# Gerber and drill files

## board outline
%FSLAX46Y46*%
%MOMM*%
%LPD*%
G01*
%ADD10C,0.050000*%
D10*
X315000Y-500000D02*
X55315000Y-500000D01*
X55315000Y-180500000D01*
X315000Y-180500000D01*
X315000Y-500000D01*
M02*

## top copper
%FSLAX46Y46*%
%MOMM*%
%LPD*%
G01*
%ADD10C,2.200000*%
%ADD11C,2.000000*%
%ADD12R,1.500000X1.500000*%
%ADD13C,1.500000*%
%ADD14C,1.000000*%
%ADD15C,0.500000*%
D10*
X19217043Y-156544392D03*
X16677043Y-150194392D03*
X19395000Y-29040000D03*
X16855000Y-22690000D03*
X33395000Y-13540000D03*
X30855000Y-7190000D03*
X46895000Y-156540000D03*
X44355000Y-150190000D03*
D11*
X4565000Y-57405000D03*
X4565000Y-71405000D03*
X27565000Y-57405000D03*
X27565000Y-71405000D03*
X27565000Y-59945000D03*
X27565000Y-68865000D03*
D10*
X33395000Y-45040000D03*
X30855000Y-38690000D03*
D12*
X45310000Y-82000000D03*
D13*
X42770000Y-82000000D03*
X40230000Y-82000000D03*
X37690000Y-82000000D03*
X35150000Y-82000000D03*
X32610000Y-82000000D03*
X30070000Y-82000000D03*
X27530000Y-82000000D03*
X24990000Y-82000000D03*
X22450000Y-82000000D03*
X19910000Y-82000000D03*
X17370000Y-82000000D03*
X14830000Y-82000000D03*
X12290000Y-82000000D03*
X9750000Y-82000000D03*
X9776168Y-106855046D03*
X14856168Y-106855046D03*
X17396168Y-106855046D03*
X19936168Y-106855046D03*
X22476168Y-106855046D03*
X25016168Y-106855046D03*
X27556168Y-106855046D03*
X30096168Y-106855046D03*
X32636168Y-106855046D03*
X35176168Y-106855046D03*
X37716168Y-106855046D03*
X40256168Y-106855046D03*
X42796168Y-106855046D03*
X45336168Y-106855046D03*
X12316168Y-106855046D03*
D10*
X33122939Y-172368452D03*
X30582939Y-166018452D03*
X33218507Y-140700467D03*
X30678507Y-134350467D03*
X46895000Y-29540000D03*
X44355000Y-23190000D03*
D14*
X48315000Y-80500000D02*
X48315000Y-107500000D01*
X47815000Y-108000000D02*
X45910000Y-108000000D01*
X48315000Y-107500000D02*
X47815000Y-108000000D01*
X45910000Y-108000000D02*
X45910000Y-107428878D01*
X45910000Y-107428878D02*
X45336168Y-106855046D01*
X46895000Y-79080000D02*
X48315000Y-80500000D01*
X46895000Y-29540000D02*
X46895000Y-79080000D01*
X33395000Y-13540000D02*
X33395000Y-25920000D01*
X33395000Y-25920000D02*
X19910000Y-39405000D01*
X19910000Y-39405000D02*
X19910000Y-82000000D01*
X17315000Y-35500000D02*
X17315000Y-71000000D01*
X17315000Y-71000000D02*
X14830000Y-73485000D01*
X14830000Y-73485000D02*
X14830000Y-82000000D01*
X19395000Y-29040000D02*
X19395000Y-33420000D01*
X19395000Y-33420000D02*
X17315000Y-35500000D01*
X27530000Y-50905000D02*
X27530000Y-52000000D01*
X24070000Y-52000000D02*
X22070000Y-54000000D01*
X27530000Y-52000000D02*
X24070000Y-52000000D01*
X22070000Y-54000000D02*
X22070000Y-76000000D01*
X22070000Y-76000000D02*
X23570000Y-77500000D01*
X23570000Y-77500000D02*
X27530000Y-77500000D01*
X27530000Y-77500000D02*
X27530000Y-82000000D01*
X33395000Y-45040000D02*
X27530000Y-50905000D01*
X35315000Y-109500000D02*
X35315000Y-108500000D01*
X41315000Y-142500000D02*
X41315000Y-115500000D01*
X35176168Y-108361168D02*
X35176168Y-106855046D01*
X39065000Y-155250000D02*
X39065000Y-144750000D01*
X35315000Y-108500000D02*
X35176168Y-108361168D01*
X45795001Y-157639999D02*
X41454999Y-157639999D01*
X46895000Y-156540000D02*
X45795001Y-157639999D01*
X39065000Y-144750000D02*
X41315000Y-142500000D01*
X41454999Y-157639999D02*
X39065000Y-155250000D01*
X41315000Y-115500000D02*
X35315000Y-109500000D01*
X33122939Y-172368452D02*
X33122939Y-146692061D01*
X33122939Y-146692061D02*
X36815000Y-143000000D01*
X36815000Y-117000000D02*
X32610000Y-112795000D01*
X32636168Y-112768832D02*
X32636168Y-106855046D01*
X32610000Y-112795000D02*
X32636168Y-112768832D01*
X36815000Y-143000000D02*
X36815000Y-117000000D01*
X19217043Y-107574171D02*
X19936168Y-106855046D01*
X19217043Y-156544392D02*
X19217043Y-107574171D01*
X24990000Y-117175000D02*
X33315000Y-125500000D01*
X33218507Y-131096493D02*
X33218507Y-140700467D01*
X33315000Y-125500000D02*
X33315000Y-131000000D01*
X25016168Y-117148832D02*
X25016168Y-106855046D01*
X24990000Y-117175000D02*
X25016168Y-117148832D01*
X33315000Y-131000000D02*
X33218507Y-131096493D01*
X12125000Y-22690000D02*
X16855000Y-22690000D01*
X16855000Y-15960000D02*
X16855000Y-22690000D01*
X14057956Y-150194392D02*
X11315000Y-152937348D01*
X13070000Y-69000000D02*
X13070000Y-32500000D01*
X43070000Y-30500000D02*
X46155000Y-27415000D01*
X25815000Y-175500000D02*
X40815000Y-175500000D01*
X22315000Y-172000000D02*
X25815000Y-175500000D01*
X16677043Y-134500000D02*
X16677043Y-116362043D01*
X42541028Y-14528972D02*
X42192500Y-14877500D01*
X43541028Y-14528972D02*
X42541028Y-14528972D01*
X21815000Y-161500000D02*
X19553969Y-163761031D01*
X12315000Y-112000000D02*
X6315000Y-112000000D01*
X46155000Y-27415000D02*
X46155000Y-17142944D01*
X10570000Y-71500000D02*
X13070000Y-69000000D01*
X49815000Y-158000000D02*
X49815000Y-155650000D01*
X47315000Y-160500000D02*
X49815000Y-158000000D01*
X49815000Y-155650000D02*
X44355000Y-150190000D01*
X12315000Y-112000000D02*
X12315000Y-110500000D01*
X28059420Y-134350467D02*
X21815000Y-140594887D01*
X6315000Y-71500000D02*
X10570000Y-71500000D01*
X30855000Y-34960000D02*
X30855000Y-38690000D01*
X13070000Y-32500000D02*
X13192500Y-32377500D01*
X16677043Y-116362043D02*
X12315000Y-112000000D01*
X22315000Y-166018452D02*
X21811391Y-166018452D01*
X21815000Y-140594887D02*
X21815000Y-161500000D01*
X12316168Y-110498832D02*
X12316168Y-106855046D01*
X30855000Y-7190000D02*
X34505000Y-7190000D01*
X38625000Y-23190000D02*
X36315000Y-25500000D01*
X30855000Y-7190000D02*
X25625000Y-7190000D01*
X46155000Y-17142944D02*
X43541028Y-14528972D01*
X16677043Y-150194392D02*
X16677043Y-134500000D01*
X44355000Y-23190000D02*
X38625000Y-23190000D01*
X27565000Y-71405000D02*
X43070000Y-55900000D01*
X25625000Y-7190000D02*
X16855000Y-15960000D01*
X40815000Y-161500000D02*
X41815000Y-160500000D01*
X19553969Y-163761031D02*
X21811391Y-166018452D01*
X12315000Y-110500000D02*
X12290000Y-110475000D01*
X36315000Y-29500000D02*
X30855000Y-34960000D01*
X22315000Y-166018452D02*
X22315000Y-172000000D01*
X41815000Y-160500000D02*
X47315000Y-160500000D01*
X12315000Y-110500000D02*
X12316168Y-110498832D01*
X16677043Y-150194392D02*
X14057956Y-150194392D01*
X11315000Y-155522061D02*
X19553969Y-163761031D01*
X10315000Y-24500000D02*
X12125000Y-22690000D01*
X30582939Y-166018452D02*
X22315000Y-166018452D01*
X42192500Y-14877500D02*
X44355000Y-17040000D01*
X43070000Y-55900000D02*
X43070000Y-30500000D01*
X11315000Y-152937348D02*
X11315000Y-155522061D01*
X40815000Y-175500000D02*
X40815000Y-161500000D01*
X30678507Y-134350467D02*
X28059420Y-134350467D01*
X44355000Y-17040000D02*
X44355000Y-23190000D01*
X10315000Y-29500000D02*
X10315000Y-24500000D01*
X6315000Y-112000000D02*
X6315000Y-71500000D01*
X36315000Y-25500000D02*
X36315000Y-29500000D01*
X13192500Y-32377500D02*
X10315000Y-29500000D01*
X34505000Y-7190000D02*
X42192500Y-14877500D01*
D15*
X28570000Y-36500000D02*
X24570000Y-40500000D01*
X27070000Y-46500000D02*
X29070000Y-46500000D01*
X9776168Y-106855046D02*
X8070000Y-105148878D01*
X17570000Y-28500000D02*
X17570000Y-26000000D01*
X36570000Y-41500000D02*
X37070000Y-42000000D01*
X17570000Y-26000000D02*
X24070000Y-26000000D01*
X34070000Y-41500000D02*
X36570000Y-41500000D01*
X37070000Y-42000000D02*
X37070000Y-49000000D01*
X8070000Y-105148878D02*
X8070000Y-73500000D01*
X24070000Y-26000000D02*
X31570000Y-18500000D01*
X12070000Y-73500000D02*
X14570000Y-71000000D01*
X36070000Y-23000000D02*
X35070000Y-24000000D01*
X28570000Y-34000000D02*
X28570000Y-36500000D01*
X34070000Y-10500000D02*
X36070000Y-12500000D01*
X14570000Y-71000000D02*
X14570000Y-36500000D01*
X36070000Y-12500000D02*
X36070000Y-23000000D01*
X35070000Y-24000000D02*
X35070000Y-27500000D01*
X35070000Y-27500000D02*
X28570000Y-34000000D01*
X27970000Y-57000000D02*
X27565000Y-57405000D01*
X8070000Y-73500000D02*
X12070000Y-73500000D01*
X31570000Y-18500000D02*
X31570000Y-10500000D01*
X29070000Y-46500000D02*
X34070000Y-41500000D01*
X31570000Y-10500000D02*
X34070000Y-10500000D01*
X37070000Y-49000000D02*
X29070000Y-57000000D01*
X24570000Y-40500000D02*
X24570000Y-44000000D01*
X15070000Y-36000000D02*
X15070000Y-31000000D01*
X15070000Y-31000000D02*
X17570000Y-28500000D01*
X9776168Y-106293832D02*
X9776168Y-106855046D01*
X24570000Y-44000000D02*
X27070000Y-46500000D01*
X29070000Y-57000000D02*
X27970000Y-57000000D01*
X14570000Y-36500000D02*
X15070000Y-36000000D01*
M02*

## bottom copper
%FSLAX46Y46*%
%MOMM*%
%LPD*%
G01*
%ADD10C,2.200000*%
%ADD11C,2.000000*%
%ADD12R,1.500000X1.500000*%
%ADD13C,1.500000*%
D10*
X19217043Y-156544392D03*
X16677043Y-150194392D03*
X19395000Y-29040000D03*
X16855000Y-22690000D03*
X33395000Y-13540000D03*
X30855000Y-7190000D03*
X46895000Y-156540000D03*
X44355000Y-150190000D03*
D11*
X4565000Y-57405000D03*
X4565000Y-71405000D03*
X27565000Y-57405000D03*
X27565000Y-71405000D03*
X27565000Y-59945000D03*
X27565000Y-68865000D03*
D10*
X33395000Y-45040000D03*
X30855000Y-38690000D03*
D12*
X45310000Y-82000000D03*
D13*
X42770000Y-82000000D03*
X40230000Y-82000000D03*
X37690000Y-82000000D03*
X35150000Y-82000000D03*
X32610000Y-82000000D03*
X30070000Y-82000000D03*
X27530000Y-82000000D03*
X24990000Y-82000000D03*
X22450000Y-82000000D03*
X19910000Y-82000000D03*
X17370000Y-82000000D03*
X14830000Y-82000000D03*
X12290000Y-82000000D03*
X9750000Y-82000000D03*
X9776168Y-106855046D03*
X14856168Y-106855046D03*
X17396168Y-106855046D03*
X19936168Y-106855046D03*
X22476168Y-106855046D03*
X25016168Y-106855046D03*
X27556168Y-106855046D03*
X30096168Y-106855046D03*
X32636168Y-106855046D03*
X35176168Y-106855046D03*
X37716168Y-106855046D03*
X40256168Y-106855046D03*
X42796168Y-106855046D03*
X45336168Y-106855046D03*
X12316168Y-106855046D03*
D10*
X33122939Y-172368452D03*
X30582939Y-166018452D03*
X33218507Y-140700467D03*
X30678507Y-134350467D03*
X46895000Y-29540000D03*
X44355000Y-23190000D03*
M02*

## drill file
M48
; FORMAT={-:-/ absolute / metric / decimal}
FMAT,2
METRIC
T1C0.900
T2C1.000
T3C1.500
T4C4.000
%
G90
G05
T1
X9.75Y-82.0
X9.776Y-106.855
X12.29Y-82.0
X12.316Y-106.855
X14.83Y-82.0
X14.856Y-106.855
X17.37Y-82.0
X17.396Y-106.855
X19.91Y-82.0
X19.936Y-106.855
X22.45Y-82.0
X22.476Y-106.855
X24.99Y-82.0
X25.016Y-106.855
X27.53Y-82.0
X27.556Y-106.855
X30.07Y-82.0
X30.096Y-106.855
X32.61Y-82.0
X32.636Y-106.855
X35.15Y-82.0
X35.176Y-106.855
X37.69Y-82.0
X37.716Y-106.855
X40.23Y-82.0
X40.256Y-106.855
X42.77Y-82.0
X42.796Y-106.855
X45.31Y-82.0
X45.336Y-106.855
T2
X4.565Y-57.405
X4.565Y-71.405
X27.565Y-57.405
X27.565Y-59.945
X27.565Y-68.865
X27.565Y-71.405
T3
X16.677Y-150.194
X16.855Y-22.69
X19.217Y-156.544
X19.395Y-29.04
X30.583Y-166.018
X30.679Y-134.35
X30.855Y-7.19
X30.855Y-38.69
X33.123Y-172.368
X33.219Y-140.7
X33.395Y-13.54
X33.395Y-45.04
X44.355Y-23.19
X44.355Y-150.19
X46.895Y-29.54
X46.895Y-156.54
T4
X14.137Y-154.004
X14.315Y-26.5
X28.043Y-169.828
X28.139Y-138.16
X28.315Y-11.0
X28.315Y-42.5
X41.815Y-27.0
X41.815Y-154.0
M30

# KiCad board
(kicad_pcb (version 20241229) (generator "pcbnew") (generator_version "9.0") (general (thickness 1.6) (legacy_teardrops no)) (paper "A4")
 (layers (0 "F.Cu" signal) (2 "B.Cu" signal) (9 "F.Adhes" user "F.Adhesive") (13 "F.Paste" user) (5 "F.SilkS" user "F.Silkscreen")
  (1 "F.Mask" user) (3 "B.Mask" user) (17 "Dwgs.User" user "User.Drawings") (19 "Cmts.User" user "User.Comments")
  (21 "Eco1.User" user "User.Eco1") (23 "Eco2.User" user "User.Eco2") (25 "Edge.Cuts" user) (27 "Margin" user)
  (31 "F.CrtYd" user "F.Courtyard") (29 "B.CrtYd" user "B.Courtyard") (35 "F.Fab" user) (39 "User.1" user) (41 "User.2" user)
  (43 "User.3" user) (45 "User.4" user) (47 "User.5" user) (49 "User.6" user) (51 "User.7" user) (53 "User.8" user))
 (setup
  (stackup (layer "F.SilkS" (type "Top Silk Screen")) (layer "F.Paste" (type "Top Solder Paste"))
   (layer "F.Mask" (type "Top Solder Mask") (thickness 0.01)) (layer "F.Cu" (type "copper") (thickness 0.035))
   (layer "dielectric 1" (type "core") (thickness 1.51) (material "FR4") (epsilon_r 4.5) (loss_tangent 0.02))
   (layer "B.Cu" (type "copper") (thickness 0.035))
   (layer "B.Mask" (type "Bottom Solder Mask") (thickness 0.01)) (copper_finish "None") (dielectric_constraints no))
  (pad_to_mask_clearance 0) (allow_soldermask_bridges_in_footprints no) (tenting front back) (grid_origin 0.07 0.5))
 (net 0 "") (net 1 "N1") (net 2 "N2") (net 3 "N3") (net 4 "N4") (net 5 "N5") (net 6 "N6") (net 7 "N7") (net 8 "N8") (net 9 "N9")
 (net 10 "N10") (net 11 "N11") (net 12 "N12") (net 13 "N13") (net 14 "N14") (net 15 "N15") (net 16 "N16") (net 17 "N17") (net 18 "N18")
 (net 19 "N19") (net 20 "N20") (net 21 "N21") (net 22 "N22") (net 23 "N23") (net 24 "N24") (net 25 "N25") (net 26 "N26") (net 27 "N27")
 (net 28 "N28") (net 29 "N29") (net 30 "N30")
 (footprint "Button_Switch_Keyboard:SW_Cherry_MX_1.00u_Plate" (layer "F.Cu") (at 19.217043 156.544392 -90)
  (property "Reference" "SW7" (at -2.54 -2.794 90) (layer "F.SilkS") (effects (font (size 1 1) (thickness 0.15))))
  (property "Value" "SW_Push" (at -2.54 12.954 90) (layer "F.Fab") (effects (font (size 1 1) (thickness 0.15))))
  (pad "" np_thru_hole circle (at -2.54 5.08 270) (size 4 4) (drill 4) (layers "*.Cu" "*.Mask"))
  (pad "1" thru_hole circle (at 0 0 270) (size 2.2 2.2) (drill 1.5) (layers "*.Cu" "*.Mask") (remove_unused_layers no) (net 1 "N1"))
  (pad "2" thru_hole circle (at -6.35 2.54 270) (size 2.2 2.2) (drill 1.5) (layers "*.Cu" "*.Mask") (remove_unused_layers no) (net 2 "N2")))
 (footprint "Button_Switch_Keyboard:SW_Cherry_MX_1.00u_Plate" (layer "F.Cu") (at 19.395 29.04 -90)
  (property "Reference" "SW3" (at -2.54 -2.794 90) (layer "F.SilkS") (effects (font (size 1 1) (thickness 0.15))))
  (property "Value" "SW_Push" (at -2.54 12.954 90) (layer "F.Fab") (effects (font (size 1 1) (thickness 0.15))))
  (pad "" np_thru_hole circle (at -2.54 5.08 270) (size 4 4) (drill 4) (layers "*.Cu" "*.Mask"))
  (pad "1" thru_hole circle (at 0 0 270) (size 2.2 2.2) (drill 1.5) (layers "*.Cu" "*.Mask") (remove_unused_layers no) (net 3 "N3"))
  (pad "2" thru_hole circle (at -6.35 2.54 270) (size 2.2 2.2) (drill 1.5) (layers "*.Cu" "*.Mask") (remove_unused_layers no) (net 2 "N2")))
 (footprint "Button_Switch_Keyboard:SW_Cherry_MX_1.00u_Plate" (layer "F.Cu") (at 33.395 13.54 -90)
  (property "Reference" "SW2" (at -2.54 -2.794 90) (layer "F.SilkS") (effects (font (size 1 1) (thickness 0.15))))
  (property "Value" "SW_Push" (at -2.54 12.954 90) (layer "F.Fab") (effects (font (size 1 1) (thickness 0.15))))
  (pad "" np_thru_hole circle (at -2.54 5.08 270) (size 4 4) (drill 4) (layers "*.Cu" "*.Mask"))
  (pad "1" thru_hole circle (at 0 0 270) (size 2.2 2.2) (drill 1.5) (layers "*.Cu" "*.Mask") (remove_unused_layers no) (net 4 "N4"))
  (pad "2" thru_hole circle (at -6.35 2.54 270) (size 2.2 2.2) (drill 1.5) (layers "*.Cu" "*.Mask") (remove_unused_layers no) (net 2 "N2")))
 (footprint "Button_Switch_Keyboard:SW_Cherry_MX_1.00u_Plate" (layer "F.Cu") (at 46.895 156.54 -90)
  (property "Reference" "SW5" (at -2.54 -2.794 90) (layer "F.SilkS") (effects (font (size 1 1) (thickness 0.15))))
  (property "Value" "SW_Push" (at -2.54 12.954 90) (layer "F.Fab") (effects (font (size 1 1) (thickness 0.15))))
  (pad "" np_thru_hole circle (at -2.54 5.08 270) (size 4 4) (drill 4) (layers "*.Cu" "*.Mask"))
  (pad "1" thru_hole circle (at 0 0 270) (size 2.2 2.2) (drill 1.5) (layers "*.Cu" "*.Mask") (remove_unused_layers no) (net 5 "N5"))
  (pad "2" thru_hole circle (at -6.35 2.54 270) (size 2.2 2.2) (drill 1.5) (layers "*.Cu" "*.Mask") (remove_unused_layers no) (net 2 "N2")))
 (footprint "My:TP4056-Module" (layer "F.Cu") (at 2.065 73.005)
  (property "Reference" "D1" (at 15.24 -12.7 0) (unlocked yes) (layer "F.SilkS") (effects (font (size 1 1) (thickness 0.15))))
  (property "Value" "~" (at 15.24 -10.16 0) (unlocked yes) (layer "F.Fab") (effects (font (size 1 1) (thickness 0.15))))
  (pad "1" thru_hole circle (at 2.5 -15.6) (size 2 2) (drill 1) (layers "*.Cu" "*.Mask") (remove_unused_layers no))
  (pad "2" thru_hole circle (at 2.5 -1.6) (size 2 2) (drill 1) (layers "*.Cu" "*.Mask") (remove_unused_layers no))
  (pad "3" thru_hole circle (at 25.5 -15.6) (size 2 2) (drill 1) (layers "*.Cu" "*.Mask") (remove_unused_layers no) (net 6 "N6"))
  (pad "4" thru_hole circle (at 25.5 -1.6) (size 2 2) (drill 1) (layers "*.Cu" "*.Mask") (remove_unused_layers no) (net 2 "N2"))
  (pad "5" thru_hole circle (at 25.5 -13.06) (size 2 2) (drill 1) (layers "*.Cu" "*.Mask") (remove_unused_layers no))
  (pad "6" thru_hole circle (at 25.5 -4.14) (size 2 2) (drill 1) (layers "*.Cu" "*.Mask") (remove_unused_layers no)))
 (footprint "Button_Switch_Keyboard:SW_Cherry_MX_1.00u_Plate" (layer "F.Cu") (at 33.395 45.04 -90)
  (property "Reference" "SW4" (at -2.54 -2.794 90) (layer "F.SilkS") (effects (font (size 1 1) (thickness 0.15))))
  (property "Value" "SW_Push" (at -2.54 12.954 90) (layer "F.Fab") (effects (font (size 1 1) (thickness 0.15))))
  (pad "" np_thru_hole circle (at -2.54 5.08 270) (size 4 4) (drill 4) (layers "*.Cu" "*.Mask"))
  (pad "1" thru_hole circle (at 0 0 270) (size 2.2 2.2) (drill 1.5) (layers "*.Cu" "*.Mask") (remove_unused_layers no) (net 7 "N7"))
  (pad "2" thru_hole circle (at -6.35 2.54 270) (size 2.2 2.2) (drill 1.5) (layers "*.Cu" "*.Mask") (remove_unused_layers no) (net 2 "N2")))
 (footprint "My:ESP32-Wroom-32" (layer "F.Cu") (at 45.31 82 -90)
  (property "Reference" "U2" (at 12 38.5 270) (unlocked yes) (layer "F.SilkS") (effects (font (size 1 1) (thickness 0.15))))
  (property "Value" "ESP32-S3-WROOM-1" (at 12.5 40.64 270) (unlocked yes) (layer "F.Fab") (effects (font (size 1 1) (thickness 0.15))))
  (pad "1" thru_hole rect (at 0 0 270) (size 1.5 1.5) (drill 0.9) (layers "*.Cu" "*.Mask") (remove_unused_layers yes) (keep_end_layers yes)
   (zone_layer_connections) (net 2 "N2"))
  (pad "2" thru_hole circle (at 0 2.54 270) (size 1.5 1.5) (drill 0.9) (layers "*.Cu" "*.Mask") (remove_unused_layers yes)
   (keep_end_layers yes) (zone_layer_connections) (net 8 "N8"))
  (pad "3" thru_hole circle (at 0 5.08 270) (size 1.5 1.5) (drill 0.9) (layers "*.Cu" "*.Mask") (remove_unused_layers yes)
   (keep_end_layers yes) (zone_layer_connections) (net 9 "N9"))
  (pad "4" thru_hole circle (at 0 7.62 270) (size 1.5 1.5) (drill 0.9) (layers "*.Cu" "*.Mask") (remove_unused_layers yes)
   (keep_end_layers yes) (zone_layer_connections) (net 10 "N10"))
  (pad "5" thru_hole circle (at 0 10.16 270) (size 1.5 1.5) (drill 0.9) (layers "*.Cu" "*.Mask") (remove_unused_layers yes)
   (keep_end_layers yes) (zone_layer_connections) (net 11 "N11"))
  (pad "6" thru_hole circle (at 0 12.7 270) (size 1.5 1.5) (drill 0.9) (layers "*.Cu" "*.Mask") (remove_unused_layers yes)
   (keep_end_layers yes) (zone_layer_connections) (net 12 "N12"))
  (pad "7" thru_hole circle (at 0 15.24 270) (size 1.5 1.5) (drill 0.9) (layers "*.Cu" "*.Mask") (remove_unused_layers yes)
   (keep_end_layers yes) (zone_layer_connections) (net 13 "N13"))
  (pad "8" thru_hole circle (at 0 17.78 270) (size 1.5 1.5) (drill 0.9) (layers "*.Cu" "*.Mask") (remove_unused_layers yes)
   (keep_end_layers yes) (zone_layer_connections) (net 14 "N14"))
  (pad "9" thru_hole circle (at 0 20.32 270) (size 1.5 1.5) (drill 0.9) (layers "*.Cu" "*.Mask") (remove_unused_layers yes)
   (keep_end_layers yes) (zone_layer_connections) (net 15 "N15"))
  (pad "10" thru_hole circle (at 0 22.86 270) (size 1.5 1.5) (drill 0.9) (layers "*.Cu" "*.Mask") (remove_unused_layers yes)
   (keep_end_layers yes) (zone_layer_connections) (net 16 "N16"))
  (pad "11" thru_hole circle (at 0 25.4 270) (size 1.5 1.5) (drill 0.9) (layers "*.Cu" "*.Mask") (remove_unused_layers yes)
   (keep_end_layers yes) (zone_layer_connections) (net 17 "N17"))
  (pad "12" thru_hole circle (at 0 27.94 270) (size 1.5 1.5) (drill 0.9) (layers "*.Cu" "*.Mask") (remove_unused_layers yes)
   (keep_end_layers yes) (zone_layer_connections) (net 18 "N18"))
  (pad "13" thru_hole circle (at 0 30.48 270) (size 1.5 1.5) (drill 0.9) (layers "*.Cu" "*.Mask") (remove_unused_layers yes)
   (keep_end_layers yes) (zone_layer_connections) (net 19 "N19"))
  (pad "14" thru_hole circle (at 0 33.02 270) (size 1.5 1.5) (drill 0.9) (layers "*.Cu" "*.Mask") (remove_unused_layers yes)
   (keep_end_layers yes) (zone_layer_connections) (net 5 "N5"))
  (pad "15" thru_hole circle (at 0 35.56 270) (size 1.5 1.5) (drill 0.9) (layers "*.Cu" "*.Mask") (remove_unused_layers yes)
   (keep_end_layers yes) (zone_layer_connections) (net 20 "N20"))
  (pad "16" thru_hole circle (at 24.855046 35.533832 270) (size 1.5 1.5) (drill 0.9) (layers "*.Cu" "*.Mask") (remove_unused_layers yes)
   (keep_end_layers yes) (zone_layer_connections) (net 6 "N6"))
  (pad "18" thru_hole circle (at 24.855046 30.453832 270) (size 1.5 1.5) (drill 0.9) (layers "*.Cu" "*.Mask") (remove_unused_layers yes)
   (keep_end_layers yes) (zone_layer_connections) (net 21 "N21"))
  (pad "19" thru_hole circle (at 24.855046 27.913832 270) (size 1.5 1.5) (drill 0.9) (layers "*.Cu" "*.Mask") (remove_unused_layers yes)
   (keep_end_layers yes) (zone_layer_connections) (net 4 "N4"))
  (pad "20" thru_hole circle (at 24.855046 25.373832 270) (size 1.5 1.5) (drill 0.9) (layers "*.Cu" "*.Mask") (remove_unused_layers yes)
   (keep_end_layers yes) (zone_layer_connections) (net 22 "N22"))
  (pad "21" thru_hole circle (at 24.855046 22.833832 270) (size 1.5 1.5) (drill 0.9) (layers "*.Cu" "*.Mask") (remove_unused_layers yes)
   (keep_end_layers yes) (zone_layer_connections) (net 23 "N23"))
  (pad "22" thru_hole circle (at 24.855046 20.293832 270) (size 1.5 1.5) (drill 0.9) (layers "*.Cu" "*.Mask") (remove_unused_layers yes)
   (keep_end_layers yes) (zone_layer_connections) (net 1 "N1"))
  (pad "23" thru_hole circle (at 24.855046 17.753832 270) (size 1.5 1.5) (drill 0.9) (layers "*.Cu" "*.Mask") (remove_unused_layers yes)
   (keep_end_layers yes) (zone_layer_connections) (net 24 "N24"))
  (pad "24" thru_hole circle (at 24.855046 15.213832 270) (size 1.5 1.5) (drill 0.9) (layers "*.Cu" "*.Mask") (remove_unused_layers yes)
   (keep_end_layers yes) (zone_layer_connections) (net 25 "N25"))
  (pad "25" thru_hole circle (at 24.855046 12.673832 270) (size 1.5 1.5) (drill 0.9) (layers "*.Cu" "*.Mask") (remove_unused_layers yes)
   (keep_end_layers yes) (zone_layer_connections) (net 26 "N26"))
  (pad "26" thru_hole circle (at 24.855046 10.133832 270) (size 1.5 1.5) (drill 0.9) (layers "*.Cu" "*.Mask") (remove_unused_layers yes)
   (keep_end_layers yes) (zone_layer_connections) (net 6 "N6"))
  (pad "27" thru_hole circle (at 24.855046 7.593832 270) (size 1.5 1.5) (drill 0.9) (layers "*.Cu" "*.Mask") (remove_unused_layers yes)
   (keep_end_layers yes) (zone_layer_connections) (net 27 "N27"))
  (pad "28" thru_hole circle (at 24.855046 5.053832 270) (size 1.5 1.5) (drill 0.9) (layers "*.Cu" "*.Mask") (remove_unused_layers yes)
   (keep_end_layers yes) (zone_layer_connections) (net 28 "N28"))
  (pad "29" thru_hole circle (at 24.855046 2.513832 270) (size 1.5 1.5) (drill 0.9) (layers "*.Cu" "*.Mask") (remove_unused_layers yes)
   (keep_end_layers yes) (zone_layer_connections) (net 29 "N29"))
  (pad "30" thru_hole circle (at 24.855046 -0.026168 270) (size 1.5 1.5) (drill 0.9) (layers "*.Cu" "*.Mask") (remove_unused_layers yes)
   (keep_end_layers yes) (zone_layer_connections) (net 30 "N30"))
  (pad "GND" thru_hole circle (at 24.855046 32.993832 270) (size 1.5 1.5) (drill 0.9) (layers "*.Cu" "*.Mask") (remove_unused_layers yes)
   (keep_end_layers yes) (zone_layer_connections) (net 2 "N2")))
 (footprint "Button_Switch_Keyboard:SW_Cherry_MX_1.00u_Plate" (layer "F.Cu") (at 33.122939 172.368452 -90)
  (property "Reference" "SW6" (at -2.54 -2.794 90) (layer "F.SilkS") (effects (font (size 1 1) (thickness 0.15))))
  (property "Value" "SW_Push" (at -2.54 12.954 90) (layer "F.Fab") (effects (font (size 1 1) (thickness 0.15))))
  (pad "" np_thru_hole circle (at -2.54 5.08 270) (size 4 4) (drill 4) (layers "*.Cu" "*.Mask"))
  (pad "1" thru_hole circle (at 0 0 270) (size 2.2 2.2) (drill 1.5) (layers "*.Cu" "*.Mask") (remove_unused_layers no) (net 19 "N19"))
  (pad "2" thru_hole circle (at -6.35 2.54 270) (size 2.2 2.2) (drill 1.5) (layers "*.Cu" "*.Mask") (remove_unused_layers no) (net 2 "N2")))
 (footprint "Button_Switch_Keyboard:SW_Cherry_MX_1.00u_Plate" (layer "F.Cu") (at 33.218507 140.700467 -90)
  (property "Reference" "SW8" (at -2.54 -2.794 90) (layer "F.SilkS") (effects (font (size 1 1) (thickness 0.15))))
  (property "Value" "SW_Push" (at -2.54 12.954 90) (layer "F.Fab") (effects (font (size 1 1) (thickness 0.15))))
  (pad "" np_thru_hole circle (at -2.54 5.08 270) (size 4 4) (drill 4) (layers "*.Cu" "*.Mask"))
  (pad "1" thru_hole circle (at 0 0 270) (size 2.2 2.2) (drill 1.5) (layers "*.Cu" "*.Mask") (remove_unused_layers no) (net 26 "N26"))
  (pad "2" thru_hole circle (at -6.35 2.54 270) (size 2.2 2.2) (drill 1.5) (layers "*.Cu" "*.Mask") (remove_unused_layers no) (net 2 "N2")))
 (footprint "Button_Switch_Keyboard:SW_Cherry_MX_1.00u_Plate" (layer "F.Cu") (at 46.895 29.54 -90)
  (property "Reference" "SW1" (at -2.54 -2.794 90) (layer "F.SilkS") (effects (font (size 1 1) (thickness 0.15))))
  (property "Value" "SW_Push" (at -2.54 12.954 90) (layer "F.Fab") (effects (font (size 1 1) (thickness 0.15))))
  (pad "" np_thru_hole circle (at -2.54 5.08 270) (size 4 4) (drill 4) (layers "*.Cu" "*.Mask"))
  (pad "1" thru_hole circle (at 0 0 270) (size 2.2 2.2) (drill 1.5) (layers "*.Cu" "*.Mask") (remove_unused_layers no) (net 23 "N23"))
  (pad "2" thru_hole circle (at -6.35 2.54 270) (size 2.2 2.2) (drill 1.5) (layers "*.Cu" "*.Mask") (remove_unused_layers no) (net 2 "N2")))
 (gr_rect (start 0.315 0.5) (end 55.315 180.5) (stroke (width 0.05) (type default)) (fill no) (locked yes) (layer "Edge.Cuts"))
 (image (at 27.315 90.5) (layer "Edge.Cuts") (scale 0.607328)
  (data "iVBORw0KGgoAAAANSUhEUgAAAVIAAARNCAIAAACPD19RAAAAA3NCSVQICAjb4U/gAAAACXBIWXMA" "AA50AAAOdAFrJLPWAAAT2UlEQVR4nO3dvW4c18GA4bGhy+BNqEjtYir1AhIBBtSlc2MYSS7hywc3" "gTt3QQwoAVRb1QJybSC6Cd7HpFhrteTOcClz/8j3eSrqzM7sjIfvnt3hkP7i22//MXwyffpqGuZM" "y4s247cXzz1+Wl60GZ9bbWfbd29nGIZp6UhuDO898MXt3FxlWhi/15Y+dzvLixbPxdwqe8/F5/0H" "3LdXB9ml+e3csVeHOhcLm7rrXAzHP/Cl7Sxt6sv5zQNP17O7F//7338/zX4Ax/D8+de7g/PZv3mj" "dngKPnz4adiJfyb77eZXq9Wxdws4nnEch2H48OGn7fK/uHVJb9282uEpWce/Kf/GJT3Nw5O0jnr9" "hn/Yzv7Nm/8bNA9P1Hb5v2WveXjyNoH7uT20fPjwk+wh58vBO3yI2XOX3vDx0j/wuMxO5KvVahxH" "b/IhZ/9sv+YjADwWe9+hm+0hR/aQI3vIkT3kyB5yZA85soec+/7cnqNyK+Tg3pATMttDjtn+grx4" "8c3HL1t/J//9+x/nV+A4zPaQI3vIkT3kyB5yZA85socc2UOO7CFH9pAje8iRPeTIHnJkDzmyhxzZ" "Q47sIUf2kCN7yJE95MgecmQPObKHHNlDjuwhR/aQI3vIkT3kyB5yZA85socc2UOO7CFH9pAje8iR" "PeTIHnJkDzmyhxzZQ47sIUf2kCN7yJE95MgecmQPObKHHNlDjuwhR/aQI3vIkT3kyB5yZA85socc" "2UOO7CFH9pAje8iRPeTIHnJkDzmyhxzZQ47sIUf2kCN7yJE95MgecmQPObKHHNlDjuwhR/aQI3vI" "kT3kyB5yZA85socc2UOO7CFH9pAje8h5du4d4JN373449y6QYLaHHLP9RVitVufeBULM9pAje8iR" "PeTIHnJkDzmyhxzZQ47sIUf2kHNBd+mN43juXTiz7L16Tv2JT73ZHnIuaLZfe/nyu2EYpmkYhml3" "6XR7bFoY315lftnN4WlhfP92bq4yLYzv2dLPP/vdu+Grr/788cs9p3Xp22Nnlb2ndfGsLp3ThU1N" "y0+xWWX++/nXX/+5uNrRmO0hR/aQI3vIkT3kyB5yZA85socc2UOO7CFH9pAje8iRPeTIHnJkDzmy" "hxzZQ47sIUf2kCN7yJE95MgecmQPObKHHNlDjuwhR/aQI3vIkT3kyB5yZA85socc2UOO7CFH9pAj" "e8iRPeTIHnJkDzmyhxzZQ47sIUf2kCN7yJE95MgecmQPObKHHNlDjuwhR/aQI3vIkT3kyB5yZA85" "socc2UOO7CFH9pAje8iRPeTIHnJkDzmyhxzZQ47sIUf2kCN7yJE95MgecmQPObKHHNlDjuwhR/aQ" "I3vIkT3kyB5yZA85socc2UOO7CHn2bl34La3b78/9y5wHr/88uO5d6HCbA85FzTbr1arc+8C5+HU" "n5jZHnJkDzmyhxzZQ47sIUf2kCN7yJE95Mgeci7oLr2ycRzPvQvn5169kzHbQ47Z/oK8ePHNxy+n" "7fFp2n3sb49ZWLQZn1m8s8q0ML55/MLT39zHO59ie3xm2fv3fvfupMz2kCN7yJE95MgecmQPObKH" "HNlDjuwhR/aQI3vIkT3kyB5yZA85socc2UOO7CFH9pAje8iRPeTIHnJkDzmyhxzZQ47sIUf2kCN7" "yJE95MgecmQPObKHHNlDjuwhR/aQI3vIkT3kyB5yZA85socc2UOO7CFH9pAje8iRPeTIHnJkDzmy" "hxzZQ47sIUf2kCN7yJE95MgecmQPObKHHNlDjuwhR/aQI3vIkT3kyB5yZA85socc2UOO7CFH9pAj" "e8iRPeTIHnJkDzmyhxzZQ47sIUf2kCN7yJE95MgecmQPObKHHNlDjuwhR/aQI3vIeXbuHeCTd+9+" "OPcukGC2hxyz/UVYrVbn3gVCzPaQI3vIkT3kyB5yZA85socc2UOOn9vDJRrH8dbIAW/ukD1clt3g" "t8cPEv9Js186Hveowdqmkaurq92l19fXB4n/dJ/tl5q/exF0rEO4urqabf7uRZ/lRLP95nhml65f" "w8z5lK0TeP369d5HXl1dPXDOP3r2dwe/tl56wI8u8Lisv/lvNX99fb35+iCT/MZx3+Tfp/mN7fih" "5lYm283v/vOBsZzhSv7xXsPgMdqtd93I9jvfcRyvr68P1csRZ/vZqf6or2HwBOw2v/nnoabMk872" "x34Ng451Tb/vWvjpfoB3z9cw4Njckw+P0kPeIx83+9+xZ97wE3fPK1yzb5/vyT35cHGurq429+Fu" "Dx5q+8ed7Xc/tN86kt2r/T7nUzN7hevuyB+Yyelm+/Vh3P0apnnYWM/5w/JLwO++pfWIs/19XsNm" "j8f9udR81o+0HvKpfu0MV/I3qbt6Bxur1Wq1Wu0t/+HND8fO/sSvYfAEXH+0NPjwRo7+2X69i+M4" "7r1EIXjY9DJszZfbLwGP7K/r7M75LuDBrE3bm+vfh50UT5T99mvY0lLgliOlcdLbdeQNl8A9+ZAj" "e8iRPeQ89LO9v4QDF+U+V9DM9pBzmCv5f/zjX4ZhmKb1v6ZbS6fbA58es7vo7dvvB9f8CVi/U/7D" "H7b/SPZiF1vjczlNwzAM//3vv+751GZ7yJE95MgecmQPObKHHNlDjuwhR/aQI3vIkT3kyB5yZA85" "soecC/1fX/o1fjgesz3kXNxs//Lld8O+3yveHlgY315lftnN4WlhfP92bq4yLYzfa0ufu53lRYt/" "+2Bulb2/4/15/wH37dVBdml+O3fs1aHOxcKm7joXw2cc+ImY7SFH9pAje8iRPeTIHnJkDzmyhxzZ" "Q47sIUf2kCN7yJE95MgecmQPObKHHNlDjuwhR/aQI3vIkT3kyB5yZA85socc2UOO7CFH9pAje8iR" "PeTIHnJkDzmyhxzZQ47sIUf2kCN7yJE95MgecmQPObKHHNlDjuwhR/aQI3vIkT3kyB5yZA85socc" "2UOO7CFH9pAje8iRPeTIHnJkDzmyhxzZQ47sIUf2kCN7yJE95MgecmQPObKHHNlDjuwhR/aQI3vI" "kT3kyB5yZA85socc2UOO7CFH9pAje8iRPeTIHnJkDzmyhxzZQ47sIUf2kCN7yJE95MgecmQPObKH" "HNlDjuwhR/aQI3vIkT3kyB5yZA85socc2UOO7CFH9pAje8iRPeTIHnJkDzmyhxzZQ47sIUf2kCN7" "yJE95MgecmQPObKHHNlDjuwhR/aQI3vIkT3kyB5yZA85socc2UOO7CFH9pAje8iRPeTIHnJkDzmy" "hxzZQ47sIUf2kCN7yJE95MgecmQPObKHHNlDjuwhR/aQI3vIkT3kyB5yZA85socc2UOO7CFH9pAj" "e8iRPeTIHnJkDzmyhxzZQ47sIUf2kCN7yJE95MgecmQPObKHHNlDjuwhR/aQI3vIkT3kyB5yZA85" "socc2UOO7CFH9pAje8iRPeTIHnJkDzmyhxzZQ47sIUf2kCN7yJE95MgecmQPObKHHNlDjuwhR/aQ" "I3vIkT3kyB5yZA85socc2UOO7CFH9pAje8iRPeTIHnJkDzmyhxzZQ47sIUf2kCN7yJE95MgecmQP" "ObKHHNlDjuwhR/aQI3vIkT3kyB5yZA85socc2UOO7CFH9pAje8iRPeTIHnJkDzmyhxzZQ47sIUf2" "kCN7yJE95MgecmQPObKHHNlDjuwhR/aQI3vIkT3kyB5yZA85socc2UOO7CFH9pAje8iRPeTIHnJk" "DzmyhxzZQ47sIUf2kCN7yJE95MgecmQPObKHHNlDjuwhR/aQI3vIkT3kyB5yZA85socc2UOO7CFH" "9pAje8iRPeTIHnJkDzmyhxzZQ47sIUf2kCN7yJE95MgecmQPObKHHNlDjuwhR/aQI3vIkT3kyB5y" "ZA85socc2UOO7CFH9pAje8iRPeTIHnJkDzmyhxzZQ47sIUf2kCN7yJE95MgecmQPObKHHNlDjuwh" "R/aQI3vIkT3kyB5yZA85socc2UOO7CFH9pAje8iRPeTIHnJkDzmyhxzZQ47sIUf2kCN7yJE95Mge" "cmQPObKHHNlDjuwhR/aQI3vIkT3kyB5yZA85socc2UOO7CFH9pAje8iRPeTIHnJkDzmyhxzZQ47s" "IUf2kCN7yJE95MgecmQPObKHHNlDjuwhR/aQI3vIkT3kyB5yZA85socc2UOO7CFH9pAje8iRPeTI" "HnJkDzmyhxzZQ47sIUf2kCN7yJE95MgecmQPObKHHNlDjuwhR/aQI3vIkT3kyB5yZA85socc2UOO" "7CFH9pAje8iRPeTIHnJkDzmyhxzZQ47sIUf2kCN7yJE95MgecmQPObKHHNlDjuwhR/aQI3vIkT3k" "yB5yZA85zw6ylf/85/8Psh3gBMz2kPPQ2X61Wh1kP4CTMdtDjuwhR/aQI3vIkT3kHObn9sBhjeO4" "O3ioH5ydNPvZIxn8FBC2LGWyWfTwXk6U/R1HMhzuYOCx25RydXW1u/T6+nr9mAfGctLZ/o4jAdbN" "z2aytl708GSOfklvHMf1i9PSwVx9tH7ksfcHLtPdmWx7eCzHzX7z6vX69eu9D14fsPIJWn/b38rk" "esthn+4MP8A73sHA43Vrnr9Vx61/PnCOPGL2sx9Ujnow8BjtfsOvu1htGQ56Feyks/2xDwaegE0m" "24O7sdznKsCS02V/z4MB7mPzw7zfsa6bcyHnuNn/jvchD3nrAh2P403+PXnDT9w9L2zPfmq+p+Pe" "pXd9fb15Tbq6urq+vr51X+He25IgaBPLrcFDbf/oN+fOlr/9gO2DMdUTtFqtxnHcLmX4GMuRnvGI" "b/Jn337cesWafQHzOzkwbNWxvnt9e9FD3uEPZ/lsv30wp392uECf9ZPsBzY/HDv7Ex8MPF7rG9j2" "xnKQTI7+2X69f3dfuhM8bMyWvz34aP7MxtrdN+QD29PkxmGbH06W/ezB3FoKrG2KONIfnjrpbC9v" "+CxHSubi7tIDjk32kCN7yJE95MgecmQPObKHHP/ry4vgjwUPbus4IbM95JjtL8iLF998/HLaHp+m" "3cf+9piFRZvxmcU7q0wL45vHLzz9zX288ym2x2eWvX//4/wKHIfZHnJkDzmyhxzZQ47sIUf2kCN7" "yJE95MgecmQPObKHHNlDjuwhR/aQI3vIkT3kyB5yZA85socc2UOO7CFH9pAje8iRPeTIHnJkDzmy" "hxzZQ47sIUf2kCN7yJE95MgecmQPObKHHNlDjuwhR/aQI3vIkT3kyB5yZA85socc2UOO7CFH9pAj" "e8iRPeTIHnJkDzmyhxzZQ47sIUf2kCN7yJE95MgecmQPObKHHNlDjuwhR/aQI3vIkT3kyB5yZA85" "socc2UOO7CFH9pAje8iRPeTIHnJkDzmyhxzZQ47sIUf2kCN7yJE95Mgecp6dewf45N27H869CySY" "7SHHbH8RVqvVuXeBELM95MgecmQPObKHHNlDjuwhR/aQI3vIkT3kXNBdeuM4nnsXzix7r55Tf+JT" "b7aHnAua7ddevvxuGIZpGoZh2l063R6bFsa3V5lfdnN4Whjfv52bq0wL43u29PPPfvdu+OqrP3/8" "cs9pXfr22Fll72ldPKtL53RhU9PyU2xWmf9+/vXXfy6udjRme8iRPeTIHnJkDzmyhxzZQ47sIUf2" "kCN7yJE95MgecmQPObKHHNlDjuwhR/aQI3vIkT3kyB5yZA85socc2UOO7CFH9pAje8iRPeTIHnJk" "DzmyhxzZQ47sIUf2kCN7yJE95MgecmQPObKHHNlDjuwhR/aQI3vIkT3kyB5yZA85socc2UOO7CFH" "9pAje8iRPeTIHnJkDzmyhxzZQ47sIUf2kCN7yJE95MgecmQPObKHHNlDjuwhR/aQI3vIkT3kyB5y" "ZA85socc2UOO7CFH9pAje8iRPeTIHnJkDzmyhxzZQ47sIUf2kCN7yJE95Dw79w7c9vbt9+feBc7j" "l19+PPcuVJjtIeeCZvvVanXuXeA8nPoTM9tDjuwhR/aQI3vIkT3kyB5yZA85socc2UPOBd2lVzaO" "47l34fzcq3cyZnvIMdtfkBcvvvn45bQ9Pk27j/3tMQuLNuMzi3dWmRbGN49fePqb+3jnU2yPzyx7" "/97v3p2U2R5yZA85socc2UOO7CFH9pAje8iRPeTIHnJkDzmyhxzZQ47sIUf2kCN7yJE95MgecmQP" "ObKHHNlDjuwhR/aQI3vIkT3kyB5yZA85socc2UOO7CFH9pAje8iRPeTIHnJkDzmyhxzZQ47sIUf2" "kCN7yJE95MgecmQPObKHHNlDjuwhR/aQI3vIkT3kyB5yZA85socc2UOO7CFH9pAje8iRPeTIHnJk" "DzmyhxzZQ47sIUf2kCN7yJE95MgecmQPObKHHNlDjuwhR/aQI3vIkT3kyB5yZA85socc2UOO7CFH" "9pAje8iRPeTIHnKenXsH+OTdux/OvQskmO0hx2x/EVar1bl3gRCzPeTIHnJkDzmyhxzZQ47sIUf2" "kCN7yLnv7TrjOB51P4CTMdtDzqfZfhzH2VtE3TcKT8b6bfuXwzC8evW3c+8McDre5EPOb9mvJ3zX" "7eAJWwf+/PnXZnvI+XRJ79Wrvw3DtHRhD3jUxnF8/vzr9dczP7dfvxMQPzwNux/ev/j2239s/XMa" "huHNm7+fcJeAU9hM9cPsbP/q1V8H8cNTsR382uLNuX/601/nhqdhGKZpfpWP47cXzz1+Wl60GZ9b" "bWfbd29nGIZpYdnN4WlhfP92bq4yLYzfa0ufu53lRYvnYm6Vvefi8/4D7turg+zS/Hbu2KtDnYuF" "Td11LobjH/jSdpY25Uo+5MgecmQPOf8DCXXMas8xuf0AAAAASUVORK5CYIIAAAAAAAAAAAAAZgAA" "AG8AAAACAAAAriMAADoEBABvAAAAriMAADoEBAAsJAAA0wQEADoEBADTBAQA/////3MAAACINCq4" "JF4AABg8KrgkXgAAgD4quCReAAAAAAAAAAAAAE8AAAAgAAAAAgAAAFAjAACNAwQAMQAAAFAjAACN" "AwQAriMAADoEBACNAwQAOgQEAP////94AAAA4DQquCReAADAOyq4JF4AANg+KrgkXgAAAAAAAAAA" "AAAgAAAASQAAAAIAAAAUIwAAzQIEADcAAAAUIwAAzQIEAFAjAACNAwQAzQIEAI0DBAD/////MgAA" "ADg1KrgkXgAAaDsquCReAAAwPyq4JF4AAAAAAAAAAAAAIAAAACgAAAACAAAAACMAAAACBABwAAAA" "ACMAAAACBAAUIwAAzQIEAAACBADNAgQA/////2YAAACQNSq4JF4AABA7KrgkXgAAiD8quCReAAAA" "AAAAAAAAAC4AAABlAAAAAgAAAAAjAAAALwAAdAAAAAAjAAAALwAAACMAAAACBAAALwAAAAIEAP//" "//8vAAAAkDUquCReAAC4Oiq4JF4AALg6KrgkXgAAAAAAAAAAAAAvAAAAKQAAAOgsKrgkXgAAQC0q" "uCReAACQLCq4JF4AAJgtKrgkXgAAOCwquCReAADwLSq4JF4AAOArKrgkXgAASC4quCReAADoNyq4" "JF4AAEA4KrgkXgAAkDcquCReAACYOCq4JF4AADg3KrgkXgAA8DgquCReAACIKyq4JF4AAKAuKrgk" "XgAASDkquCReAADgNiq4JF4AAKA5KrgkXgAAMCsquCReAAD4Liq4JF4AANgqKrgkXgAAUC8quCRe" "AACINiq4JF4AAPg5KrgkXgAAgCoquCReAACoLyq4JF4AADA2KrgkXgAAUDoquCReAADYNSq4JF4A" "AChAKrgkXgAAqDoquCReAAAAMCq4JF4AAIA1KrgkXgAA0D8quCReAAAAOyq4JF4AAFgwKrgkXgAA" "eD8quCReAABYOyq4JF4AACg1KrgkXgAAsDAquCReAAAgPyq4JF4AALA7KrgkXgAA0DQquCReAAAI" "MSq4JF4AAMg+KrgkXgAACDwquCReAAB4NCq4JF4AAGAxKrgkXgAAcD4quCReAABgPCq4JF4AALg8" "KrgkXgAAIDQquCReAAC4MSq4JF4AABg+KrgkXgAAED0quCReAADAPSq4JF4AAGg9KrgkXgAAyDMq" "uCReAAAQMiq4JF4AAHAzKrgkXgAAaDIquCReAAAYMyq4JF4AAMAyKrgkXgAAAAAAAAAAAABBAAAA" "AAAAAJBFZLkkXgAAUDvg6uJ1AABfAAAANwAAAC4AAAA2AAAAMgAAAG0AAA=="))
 (segment (start 48.315 80.5) (end 48.315 107.5) (width 1) (layer "F.Cu") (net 23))
 (segment (start 47.815 108) (end 45.91 108) (width 1) (layer "F.Cu") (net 23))
 (segment (start 48.315 107.5) (end 47.815 108) (width 1) (layer "F.Cu") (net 23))
 (segment (start 45.91 108) (end 45.91 107.428878) (width 1) (layer "F.Cu") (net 23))
 (segment (start 45.91 107.428878) (end 45.336168 106.855046) (width 1) (layer "F.Cu") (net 23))
 (segment (start 46.895 79.08) (end 48.315 80.5) (width 1) (layer "F.Cu") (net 23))
 (segment (start 46.895 29.54) (end 46.895 79.08) (width 1) (layer "F.Cu") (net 23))
 (segment (start 33.395 13.54) (end 33.395 25.92) (width 1) (layer "F.Cu") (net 4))
 (segment (start 33.395 25.92) (end 19.91 39.405) (width 1) (layer "F.Cu") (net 4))
 (segment (start 19.91 39.405) (end 19.91 82) (width 1) (layer "F.Cu") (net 4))
 (segment (start 17.315 35.5) (end 17.315 71) (width 1) (layer "F.Cu") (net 3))
 (segment (start 17.315 71) (end 14.83 73.485) (width 1) (layer "F.Cu") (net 3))
 (segment (start 14.83 73.485) (end 14.83 82) (width 1) (layer "F.Cu") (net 3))
 (segment (start 19.395 29.04) (end 19.395 33.42) (width 1) (layer "F.Cu") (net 3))
 (segment (start 19.395 33.42) (end 17.315 35.5) (width 1) (layer "F.Cu") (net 3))
 (segment (start 27.53 50.905) (end 27.53 52) (width 1) (layer "F.Cu") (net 7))
 (segment (start 24.07 52) (end 22.07 54) (width 1) (layer "F.Cu") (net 7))
 (segment (start 27.53 52) (end 24.07 52) (width 1) (layer "F.Cu") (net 7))
 (segment (start 22.07 54) (end 22.07 76) (width 1) (layer "F.Cu") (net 7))
 (segment (start 22.07 76) (end 23.57 77.5) (width 1) (layer "F.Cu") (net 7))
 (segment (start 23.57 77.5) (end 27.53 77.5) (width 1) (layer "F.Cu") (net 7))
 (segment (start 27.53 77.5) (end 27.53 82) (width 1) (layer "F.Cu") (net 7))
 (segment (start 33.395 45.04) (end 27.53 50.905) (width 1) (layer "F.Cu") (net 7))
 (segment (start 35.315 109.5) (end 35.315 108.5) (width 1) (layer "F.Cu") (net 5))
 (segment (start 41.315 142.5) (end 41.315 115.5) (width 1) (layer "F.Cu") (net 5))
 (segment (start 35.176168 108.361168) (end 35.176168 106.855046) (width 1) (layer "F.Cu") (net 5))
 (segment (start 39.065 155.25) (end 39.065 144.75) (width 1) (layer "F.Cu") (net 5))
 (segment (start 35.315 108.5) (end 35.176168 108.361168) (width 1) (layer "F.Cu") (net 5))
 (segment (start 45.795001 157.639999) (end 41.454999 157.639999) (width 1) (layer "F.Cu") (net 5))
 (segment (start 46.895 156.54) (end 45.795001 157.639999) (width 1) (layer "F.Cu") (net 5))
 (segment (start 39.065 144.75) (end 41.315 142.5) (width 1) (layer "F.Cu") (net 5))
 (segment (start 41.454999 157.639999) (end 39.065 155.25) (width 1) (layer "F.Cu") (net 5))
 (segment (start 41.315 115.5) (end 35.315 109.5) (width 1) (layer "F.Cu") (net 5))
 (segment (start 33.122939 172.368452) (end 33.122939 146.692061) (width 1) (layer "F.Cu") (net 19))
 (segment (start 33.122939 146.692061) (end 36.815 143) (width 1) (layer "F.Cu") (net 19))
 (segment (start 36.815 117) (end 32.61 112.795) (width 1) (layer "F.Cu") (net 19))
 (segment (start 32.636168 112.768832) (end 32.636168 106.855046) (width 1) (layer "F.Cu") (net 19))
 (segment (start 32.61 112.795) (end 32.636168 112.768832) (width 1) (layer "F.Cu") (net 19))
 (segment (start 36.815 143) (end 36.815 117) (width 1) (layer "F.Cu") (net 19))
 (segment (start 19.217043 107.574171) (end 19.936168 106.855046) (width 1) (layer "F.Cu") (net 1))
 (segment (start 19.217043 156.544392) (end 19.217043 107.574171) (width 1) (layer "F.Cu") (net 1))
 (segment (start 24.99 117.175) (end 33.315 125.5) (width 1) (layer "F.Cu") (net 26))
 (segment (start 33.218507 131.096493) (end 33.218507 140.700467) (width 1) (layer "F.Cu") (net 26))
 (segment (start 33.315 125.5) (end 33.315 131) (width 1) (layer "F.Cu") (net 26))
 (segment (start 25.016168 117.148832) (end 25.016168 106.855046) (width 1) (layer "F.Cu") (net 26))
 (segment (start 24.99 117.175) (end 25.016168 117.148832) (width 1) (layer "F.Cu") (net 26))
 (segment (start 33.315 131) (end 33.218507 131.096493) (width 1) (layer "F.Cu") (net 26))
 (segment (start 12.125 22.69) (end 16.855 22.69) (width 1) (layer "F.Cu") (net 2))
 (segment (start 16.855 15.96) (end 16.855 22.69) (width 1) (layer "F.Cu") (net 2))
 (segment (start 14.057956 150.194392) (end 11.315 152.937348) (width 1) (layer "F.Cu") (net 2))
 (segment (start 13.07 69) (end 13.07 32.5) (width 1) (layer "F.Cu") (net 2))
 (segment (start 43.07 30.5) (end 46.155 27.415) (width 1) (layer "F.Cu") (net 2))
 (segment (start 25.815 175.5) (end 40.815 175.5) (width 1) (layer "F.Cu") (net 2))
 (segment (start 22.315 172) (end 25.815 175.5) (width 1) (layer "F.Cu") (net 2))
 (segment (start 16.677043 134.5) (end 16.677043 116.362043) (width 1) (layer "F.Cu") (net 2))
 (segment (start 42.541028 14.528972) (end 42.1925 14.8775) (width 1) (layer "F.Cu") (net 2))
 (segment (start 43.541028 14.528972) (end 42.541028 14.528972) (width 1) (layer "F.Cu") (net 2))
 (segment (start 21.815 161.5) (end 19.553969 163.761031) (width 1) (layer "F.Cu") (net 2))
 (segment (start 12.315 112) (end 6.315 112) (width 1) (layer "F.Cu") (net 2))
 (segment (start 46.155 27.415) (end 46.155 17.142944) (width 1) (layer "F.Cu") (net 2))
 (segment (start 10.57 71.5) (end 13.07 69) (width 1) (layer "F.Cu") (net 2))
 (segment (start 49.815 158) (end 49.815 155.65) (width 1) (layer "F.Cu") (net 2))
 (segment (start 47.315 160.5) (end 49.815 158) (width 1) (layer "F.Cu") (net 2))
 (segment (start 49.815 155.65) (end 44.355 150.19) (width 1) (layer "F.Cu") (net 2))
 (segment (start 12.315 112) (end 12.315 110.5) (width 1) (layer "F.Cu") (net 2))
 (segment (start 28.05942 134.350467) (end 21.815 140.594887) (width 1) (layer "F.Cu") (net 2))
 (segment (start 6.315 71.5) (end 10.57 71.5) (width 1) (layer "F.Cu") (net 2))
 (segment (start 30.855 34.96) (end 30.855 38.69) (width 1) (layer "F.Cu") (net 2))
 (segment (start 13.07 32.5) (end 13.1925 32.3775) (width 1) (layer "F.Cu") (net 2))
 (segment (start 16.677043 116.362043) (end 12.315 112) (width 1) (layer "F.Cu") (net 2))
 (segment (start 22.315 166.018452) (end 21.811391 166.018452) (width 1) (layer "F.Cu") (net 2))
 (segment (start 21.815 140.594887) (end 21.815 161.5) (width 1) (layer "F.Cu") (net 2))
 (segment (start 12.316168 110.498832) (end 12.316168 106.855046) (width 1) (layer "F.Cu") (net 2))
 (segment (start 30.855 7.19) (end 34.505 7.19) (width 1) (layer "F.Cu") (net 2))
 (segment (start 38.625 23.19) (end 36.315 25.5) (width 1) (layer "F.Cu") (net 2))
 (segment (start 30.855 7.19) (end 25.625 7.19) (width 1) (layer "F.Cu") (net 2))
 (segment (start 46.155 17.142944) (end 43.541028 14.528972) (width 1) (layer "F.Cu") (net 2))
 (segment (start 16.677043 150.194392) (end 16.677043 134.5) (width 1) (layer "F.Cu") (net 2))
 (segment (start 44.355 23.19) (end 38.625 23.19) (width 1) (layer "F.Cu") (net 2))
 (segment (start 27.565 71.405) (end 43.07 55.9) (width 1) (layer "F.Cu") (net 2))
 (segment (start 25.625 7.19) (end 16.855 15.96) (width 1) (layer "F.Cu") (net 2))
 (segment (start 40.815 161.5) (end 41.815 160.5) (width 1) (layer "F.Cu") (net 2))
 (segment (start 19.553969 163.761031) (end 21.811391 166.018452) (width 1) (layer "F.Cu") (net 2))
 (segment (start 12.315 110.5) (end 12.29 110.475) (width 1) (layer "F.Cu") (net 2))
 (segment (start 36.315 29.5) (end 30.855 34.96) (width 1) (layer "F.Cu") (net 2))
 (segment (start 22.315 166.018452) (end 22.315 172) (width 1) (layer "F.Cu") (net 2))
 (segment (start 41.815 160.5) (end 47.315 160.5) (width 1) (layer "F.Cu") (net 2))
 (segment (start 12.315 110.5) (end 12.316168 110.498832) (width 1) (layer "F.Cu") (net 2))
 (segment (start 16.677043 150.194392) (end 14.057956 150.194392) (width 1) (layer "F.Cu") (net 2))
 (segment (start 11.315 155.522061) (end 19.553969 163.761031) (width 1) (layer "F.Cu") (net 2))
 (segment (start 10.315 24.5) (end 12.125 22.69) (width 1) (layer "F.Cu") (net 2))
 (segment (start 30.582939 166.018452) (end 22.315 166.018452) (width 1) (layer "F.Cu") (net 2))
 (segment (start 42.1925 14.8775) (end 44.355 17.04) (width 1) (layer "F.Cu") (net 2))
 (segment (start 43.07 55.9) (end 43.07 30.5) (width 1) (layer "F.Cu") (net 2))
 (segment (start 11.315 152.937348) (end 11.315 155.522061) (width 1) (layer "F.Cu") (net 2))
 (segment (start 40.815 175.5) (end 40.815 161.5) (width 1) (layer "F.Cu") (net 2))
 (segment (start 30.678507 134.350467) (end 28.05942 134.350467) (width 1) (layer "F.Cu") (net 2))
 (segment (start 44.355 17.04) (end 44.355 23.19) (width 1) (layer "F.Cu") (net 2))
 (segment (start 10.315 29.5) (end 10.315 24.5) (width 1) (layer "F.Cu") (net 2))
 (segment (start 6.315 112) (end 6.315 71.5) (width 1) (layer "F.Cu") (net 2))
 (segment (start 36.315 25.5) (end 36.315 29.5) (width 1) (layer "F.Cu") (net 2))
 (segment (start 13.1925 32.3775) (end 10.315 29.5) (width 1) (layer "F.Cu") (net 2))
 (segment (start 34.505 7.19) (end 42.1925 14.8775) (width 1) (layer "F.Cu") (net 2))
 (segment (start 28.57 36.5) (end 24.57 40.5) (width 0.5) (layer "F.Cu") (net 6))
 (segment (start 27.07 46.5) (end 29.07 46.5) (width 0.5) (layer "F.Cu") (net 6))
 (segment (start 9.776168 106.855046) (end 8.07 105.148878) (width 0.5) (layer "F.Cu") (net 6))
 (segment (start 17.57 28.5) (end 17.57 26) (width 0.5) (layer "F.Cu") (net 6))
 (segment (start 36.57 41.5) (end 37.07 42) (width 0.5) (layer "F.Cu") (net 6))
 (segment (start 17.57 26) (end 24.07 26) (width 0.5) (layer "F.Cu") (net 6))
 (segment (start 34.07 41.5) (end 36.57 41.5) (width 0.5) (layer "F.Cu") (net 6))
 (segment (start 37.07 42) (end 37.07 49) (width 0.5) (layer "F.Cu") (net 6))
 (segment (start 8.07 105.148878) (end 8.07 73.5) (width 0.5) (layer "F.Cu") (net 6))
 (segment (start 24.07 26) (end 31.57 18.5) (width 0.5) (layer "F.Cu") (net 6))
 (segment (start 12.07 73.5) (end 14.57 71) (width 0.5) (layer "F.Cu") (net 6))
 (segment (start 36.07 23) (end 35.07 24) (width 0.5) (layer "F.Cu") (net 6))
 (segment (start 28.57 34) (end 28.57 36.5) (width 0.5) (layer "F.Cu") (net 6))
 (segment (start 34.07 10.5) (end 36.07 12.5) (width 0.5) (layer "F.Cu") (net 6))
 (segment (start 14.57 71) (end 14.57 36.5) (width 0.5) (layer "F.Cu") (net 6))
 (segment (start 36.07 12.5) (end 36.07 23) (width 0.5) (layer "F.Cu") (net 6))
 (segment (start 35.07 24) (end 35.07 27.5) (width 0.5) (layer "F.Cu") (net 6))
 (segment (start 35.07 27.5) (end 28.57 34) (width 0.5) (layer "F.Cu") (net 6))
 (segment (start 27.97 57) (end 27.565 57.405) (width 0.5) (layer "F.Cu") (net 6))
 (segment (start 8.07 73.5) (end 12.07 73.5) (width 0.5) (layer "F.Cu") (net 6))
 (segment (start 31.57 18.5) (end 31.57 10.5) (width 0.5) (layer "F.Cu") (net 6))
 (segment (start 29.07 46.5) (end 34.07 41.5) (width 0.5) (layer "F.Cu") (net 6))
 (segment (start 31.57 10.5) (end 34.07 10.5) (width 0.5) (layer "F.Cu") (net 6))
 (segment (start 37.07 49) (end 29.07 57) (width 0.5) (layer "F.Cu") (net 6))
 (segment (start 24.57 40.5) (end 24.57 44) (width 0.5) (layer "F.Cu") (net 6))
 (segment (start 15.07 36) (end 15.07 31) (width 0.5) (layer "F.Cu") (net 6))
 (segment (start 15.07 31) (end 17.57 28.5) (width 0.5) (layer "F.Cu") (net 6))
 (segment (start 9.776168 106.293832) (end 9.776168 106.855046) (width 0.5) (layer "F.Cu") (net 6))
 (segment (start 24.57 44) (end 27.07 46.5) (width 0.5) (layer "F.Cu") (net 6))
 (segment (start 29.07 57) (end 27.97 57) (width 0.5) (layer "F.Cu") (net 6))
 (segment (start 14.57 36.5) (end 15.07 36) (width 0.5) (layer "F.Cu") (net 6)))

